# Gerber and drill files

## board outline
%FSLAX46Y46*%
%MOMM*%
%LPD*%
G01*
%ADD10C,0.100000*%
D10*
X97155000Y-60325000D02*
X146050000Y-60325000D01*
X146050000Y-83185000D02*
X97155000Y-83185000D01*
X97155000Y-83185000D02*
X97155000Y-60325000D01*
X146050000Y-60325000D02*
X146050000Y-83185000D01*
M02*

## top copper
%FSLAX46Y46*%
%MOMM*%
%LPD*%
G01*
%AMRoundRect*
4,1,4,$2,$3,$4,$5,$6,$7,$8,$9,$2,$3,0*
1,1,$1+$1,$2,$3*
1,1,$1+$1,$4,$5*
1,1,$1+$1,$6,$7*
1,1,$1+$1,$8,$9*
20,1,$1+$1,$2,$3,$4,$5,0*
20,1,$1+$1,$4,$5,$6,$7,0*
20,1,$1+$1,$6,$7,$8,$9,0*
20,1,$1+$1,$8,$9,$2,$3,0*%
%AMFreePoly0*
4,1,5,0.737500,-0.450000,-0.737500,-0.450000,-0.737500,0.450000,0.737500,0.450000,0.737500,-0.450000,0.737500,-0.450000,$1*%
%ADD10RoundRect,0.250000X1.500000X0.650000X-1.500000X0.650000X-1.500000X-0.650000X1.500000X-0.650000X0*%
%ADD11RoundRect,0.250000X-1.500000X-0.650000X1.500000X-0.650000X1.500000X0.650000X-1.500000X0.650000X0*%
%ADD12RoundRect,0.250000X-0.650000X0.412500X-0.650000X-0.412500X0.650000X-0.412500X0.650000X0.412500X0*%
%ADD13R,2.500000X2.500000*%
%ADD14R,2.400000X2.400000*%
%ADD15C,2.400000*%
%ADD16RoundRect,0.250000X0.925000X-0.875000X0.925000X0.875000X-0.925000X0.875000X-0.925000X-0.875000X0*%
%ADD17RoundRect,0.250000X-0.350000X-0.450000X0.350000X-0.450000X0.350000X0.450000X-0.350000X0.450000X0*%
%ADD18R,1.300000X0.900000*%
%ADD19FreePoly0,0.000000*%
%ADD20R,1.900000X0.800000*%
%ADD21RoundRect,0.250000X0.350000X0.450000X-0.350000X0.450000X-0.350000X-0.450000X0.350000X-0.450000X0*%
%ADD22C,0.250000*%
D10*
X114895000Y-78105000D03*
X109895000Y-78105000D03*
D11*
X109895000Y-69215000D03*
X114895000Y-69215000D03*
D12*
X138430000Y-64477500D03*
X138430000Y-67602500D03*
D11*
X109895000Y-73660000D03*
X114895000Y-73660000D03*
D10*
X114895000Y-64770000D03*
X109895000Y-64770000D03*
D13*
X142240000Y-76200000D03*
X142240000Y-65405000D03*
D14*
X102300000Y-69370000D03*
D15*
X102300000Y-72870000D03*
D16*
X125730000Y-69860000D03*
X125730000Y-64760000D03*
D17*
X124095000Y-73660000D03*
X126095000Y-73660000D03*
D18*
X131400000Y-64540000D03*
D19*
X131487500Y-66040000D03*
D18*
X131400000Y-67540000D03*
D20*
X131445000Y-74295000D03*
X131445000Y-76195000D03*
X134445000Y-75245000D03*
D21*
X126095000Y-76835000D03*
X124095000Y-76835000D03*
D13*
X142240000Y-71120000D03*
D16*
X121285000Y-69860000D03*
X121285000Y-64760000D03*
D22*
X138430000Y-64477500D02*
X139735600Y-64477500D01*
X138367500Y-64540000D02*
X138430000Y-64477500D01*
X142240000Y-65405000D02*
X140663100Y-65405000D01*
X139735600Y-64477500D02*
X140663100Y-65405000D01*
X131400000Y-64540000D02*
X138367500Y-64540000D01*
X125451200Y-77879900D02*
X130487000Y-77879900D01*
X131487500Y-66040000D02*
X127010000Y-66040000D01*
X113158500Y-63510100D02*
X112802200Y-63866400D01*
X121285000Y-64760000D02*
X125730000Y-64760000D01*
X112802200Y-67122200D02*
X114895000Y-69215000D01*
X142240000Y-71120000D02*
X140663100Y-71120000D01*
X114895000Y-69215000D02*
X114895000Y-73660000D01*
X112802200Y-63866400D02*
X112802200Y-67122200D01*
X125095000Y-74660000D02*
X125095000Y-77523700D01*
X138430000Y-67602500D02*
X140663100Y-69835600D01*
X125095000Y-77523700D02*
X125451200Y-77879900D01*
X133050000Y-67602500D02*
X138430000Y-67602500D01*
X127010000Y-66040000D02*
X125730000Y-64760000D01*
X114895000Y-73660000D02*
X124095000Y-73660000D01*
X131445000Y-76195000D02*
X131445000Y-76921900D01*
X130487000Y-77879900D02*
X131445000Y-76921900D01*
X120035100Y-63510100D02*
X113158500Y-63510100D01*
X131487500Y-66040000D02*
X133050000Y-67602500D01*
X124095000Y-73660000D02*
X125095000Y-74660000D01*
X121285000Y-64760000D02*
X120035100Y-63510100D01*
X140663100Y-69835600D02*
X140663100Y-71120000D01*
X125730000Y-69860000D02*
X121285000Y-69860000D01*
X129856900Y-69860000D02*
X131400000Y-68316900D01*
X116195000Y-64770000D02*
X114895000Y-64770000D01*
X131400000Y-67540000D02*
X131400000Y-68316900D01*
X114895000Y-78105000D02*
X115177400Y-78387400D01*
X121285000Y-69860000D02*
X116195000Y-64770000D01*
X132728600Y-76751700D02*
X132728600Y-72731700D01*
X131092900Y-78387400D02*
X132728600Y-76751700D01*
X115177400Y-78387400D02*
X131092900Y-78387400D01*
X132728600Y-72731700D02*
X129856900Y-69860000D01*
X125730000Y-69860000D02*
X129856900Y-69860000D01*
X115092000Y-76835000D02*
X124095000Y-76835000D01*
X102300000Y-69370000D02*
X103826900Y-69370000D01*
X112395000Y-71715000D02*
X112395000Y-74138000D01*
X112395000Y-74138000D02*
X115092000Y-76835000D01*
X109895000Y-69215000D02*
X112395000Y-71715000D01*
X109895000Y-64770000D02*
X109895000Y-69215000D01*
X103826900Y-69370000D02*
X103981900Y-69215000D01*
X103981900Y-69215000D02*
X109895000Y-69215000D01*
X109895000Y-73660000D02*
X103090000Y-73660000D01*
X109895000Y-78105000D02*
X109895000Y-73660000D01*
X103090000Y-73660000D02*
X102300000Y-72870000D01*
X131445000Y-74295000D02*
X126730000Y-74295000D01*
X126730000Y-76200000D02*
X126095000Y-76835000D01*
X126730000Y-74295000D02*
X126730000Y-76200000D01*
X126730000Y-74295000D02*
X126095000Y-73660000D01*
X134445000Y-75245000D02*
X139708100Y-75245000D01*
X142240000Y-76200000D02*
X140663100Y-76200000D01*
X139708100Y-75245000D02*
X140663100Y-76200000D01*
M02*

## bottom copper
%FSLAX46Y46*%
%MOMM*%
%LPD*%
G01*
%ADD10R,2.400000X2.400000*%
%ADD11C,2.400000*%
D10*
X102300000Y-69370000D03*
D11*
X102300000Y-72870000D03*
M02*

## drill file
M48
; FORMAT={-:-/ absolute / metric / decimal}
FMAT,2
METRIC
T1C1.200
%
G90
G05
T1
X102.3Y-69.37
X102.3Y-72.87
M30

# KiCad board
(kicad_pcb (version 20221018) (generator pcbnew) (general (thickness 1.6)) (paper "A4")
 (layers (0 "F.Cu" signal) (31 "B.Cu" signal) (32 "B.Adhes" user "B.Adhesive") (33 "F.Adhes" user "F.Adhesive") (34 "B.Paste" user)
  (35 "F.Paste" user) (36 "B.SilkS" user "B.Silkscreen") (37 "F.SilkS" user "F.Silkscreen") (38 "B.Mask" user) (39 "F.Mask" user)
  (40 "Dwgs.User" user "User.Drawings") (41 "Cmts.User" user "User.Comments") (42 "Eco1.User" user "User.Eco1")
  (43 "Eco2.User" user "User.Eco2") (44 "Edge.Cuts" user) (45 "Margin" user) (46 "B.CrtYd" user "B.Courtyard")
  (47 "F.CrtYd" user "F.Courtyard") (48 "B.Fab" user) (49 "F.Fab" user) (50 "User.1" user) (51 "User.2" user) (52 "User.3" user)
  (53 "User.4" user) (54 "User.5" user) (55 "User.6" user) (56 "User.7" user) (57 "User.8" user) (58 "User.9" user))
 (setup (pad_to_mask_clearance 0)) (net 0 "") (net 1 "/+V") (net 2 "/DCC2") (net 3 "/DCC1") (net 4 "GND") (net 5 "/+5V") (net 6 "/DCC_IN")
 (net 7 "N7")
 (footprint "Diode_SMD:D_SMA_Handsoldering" (layer "F.Cu") (at 112.395 78.105 180)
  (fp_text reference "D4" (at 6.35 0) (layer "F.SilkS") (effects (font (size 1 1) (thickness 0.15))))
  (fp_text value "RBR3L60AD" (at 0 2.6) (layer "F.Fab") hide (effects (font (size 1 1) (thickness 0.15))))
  (pad "1" smd roundrect (at -2.5 0 180) (size 3.5 1.8) (layers "F.Cu" "F.Paste" "F.Mask") (roundrect_rratio 0.1388888889) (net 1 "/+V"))
  (pad "2" smd roundrect (at 2.5 0 180) (size 3.5 1.8) (layers "F.Cu" "F.Paste" "F.Mask") (roundrect_rratio 0.1388888889) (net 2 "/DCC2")))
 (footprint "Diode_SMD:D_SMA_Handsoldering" (layer "F.Cu") (at 112.395 69.215)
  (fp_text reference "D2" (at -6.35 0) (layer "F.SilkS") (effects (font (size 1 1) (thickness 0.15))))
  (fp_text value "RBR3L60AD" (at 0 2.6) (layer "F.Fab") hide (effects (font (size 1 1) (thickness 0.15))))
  (pad "1" smd roundrect (at -2.5 0) (size 3.5 1.8) (layers "F.Cu" "F.Paste" "F.Mask") (roundrect_rratio 0.1388888889) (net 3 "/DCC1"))
  (pad "2" smd roundrect (at 2.5 0) (size 3.5 1.8) (layers "F.Cu" "F.Paste" "F.Mask") (roundrect_rratio 0.1388888889) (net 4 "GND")))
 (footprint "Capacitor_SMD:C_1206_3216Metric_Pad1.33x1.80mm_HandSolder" (layer "F.Cu") (at 138.43 66.04 -90)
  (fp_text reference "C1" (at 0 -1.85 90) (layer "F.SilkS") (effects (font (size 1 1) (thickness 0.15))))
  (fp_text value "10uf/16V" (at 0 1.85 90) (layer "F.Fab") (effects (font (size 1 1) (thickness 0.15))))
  (pad "1" smd roundrect (at -1.5625 0 270) (size 1.325 1.8) (layers "F.Cu" "F.Paste" "F.Mask") (roundrect_rratio 0.188679) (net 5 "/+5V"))
  (pad "2" smd roundrect (at 1.5625 0 270) (size 1.325 1.8) (layers "F.Cu" "F.Paste" "F.Mask") (roundrect_rratio 0.188679) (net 4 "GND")))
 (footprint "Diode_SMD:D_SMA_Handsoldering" (layer "F.Cu") (at 112.395 73.66)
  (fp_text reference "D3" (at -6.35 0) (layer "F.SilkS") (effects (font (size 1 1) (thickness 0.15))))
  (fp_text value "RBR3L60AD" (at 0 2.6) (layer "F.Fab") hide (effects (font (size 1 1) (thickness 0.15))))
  (pad "1" smd roundrect (at -2.5 0) (size 3.5 1.8) (layers "F.Cu" "F.Paste" "F.Mask") (roundrect_rratio 0.1388888889) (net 2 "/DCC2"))
  (pad "2" smd roundrect (at 2.5 0) (size 3.5 1.8) (layers "F.Cu" "F.Paste" "F.Mask") (roundrect_rratio 0.1388888889) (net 4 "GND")))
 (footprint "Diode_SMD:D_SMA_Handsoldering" (layer "F.Cu") (at 112.395 64.77 180)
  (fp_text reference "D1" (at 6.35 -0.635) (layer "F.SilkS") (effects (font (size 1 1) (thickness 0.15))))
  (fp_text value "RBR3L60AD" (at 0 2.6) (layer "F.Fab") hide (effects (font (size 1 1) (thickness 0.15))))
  (pad "1" smd roundrect (at -2.5 0 180) (size 3.5 1.8) (layers "F.Cu" "F.Paste" "F.Mask") (roundrect_rratio 0.1388888889) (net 1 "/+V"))
  (pad "2" smd roundrect (at 2.5 0 180) (size 3.5 1.8) (layers "F.Cu" "F.Paste" "F.Mask") (roundrect_rratio 0.1388888889) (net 3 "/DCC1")))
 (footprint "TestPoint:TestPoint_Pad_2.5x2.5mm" (layer "F.Cu") (at 142.24 76.2)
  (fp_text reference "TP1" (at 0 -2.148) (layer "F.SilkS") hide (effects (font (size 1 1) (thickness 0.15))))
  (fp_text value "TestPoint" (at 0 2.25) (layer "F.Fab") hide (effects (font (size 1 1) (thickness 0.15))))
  (pad "1" smd rect (at 0 0) (size 2.5 2.5) (layers "F.Cu" "F.Mask") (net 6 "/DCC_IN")))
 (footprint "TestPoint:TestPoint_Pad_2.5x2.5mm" (layer "F.Cu") (at 142.24 65.405)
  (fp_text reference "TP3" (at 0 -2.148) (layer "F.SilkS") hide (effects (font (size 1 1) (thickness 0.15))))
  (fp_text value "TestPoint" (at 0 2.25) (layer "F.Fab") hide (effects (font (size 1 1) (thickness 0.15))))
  (pad "1" smd rect (at 0 0) (size 2.5 2.5) (layers "F.Cu" "F.Mask") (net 5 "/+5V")))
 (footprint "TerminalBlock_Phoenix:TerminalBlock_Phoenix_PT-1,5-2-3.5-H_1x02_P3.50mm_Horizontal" (layer "F.Cu") (at 102.3 69.37 -90)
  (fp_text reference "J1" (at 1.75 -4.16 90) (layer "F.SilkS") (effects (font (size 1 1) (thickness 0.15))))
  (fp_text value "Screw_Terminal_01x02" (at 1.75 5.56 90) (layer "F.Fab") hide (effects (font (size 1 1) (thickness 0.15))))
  (pad "1" thru_hole rect (at 0 0 270) (size 2.4 2.4) (drill 1.2) (layers "*.Cu" "*.Mask") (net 3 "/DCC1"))
  (pad "2" thru_hole circle (at 3.5 0 270) (size 2.4 2.4) (drill 1.2) (layers "*.Cu" "*.Mask") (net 2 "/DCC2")))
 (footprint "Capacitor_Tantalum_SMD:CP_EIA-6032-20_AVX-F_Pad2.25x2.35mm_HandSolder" (layer "F.Cu") (at 125.73 67.31 90)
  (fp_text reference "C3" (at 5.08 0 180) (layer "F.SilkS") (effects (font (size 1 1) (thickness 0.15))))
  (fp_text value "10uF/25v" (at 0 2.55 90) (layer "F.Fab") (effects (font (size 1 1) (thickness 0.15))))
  (pad "1" smd roundrect (at -2.55 0 90) (size 2.25 2.35) (layers "F.Cu" "F.Paste" "F.Mask") (roundrect_rratio 0.111111) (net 1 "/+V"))
  (pad "2" smd roundrect (at 2.55 0 90) (size 2.25 2.35) (layers "F.Cu" "F.Paste" "F.Mask") (roundrect_rratio 0.111111) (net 4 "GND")))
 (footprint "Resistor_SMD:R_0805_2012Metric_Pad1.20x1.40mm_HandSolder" (layer "F.Cu") (at 125.095 73.66)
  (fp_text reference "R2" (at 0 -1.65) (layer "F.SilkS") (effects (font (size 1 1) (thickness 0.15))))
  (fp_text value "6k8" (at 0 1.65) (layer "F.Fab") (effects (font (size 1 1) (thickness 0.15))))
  (pad "1" smd roundrect (at -1 0) (size 1.2 1.4) (layers "F.Cu" "F.Paste" "F.Mask") (roundrect_rratio 0.208333) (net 4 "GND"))
  (pad "2" smd roundrect (at 1 0) (size 1.2 1.4) (layers "F.Cu" "F.Paste" "F.Mask") (roundrect_rratio 0.208333) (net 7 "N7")))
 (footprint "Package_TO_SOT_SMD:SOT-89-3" (layer "F.Cu") (at 133.35 66.04)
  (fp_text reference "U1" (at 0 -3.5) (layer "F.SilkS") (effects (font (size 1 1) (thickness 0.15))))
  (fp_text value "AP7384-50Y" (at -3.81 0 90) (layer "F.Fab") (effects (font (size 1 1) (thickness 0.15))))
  (pad "1" smd rect (at -1.95 -1.5) (size 1.3 0.9) (layers "F.Cu" "F.Paste" "F.Mask") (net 5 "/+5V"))
  (pad "2" smd custom (at -1.8625 0) (size 1.475 0.9) (layers "F.Cu" "F.Paste" "F.Mask") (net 4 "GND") (zone_connect 2)
   (thermal_bridge_angle 45) (options (clearance outline) (anchor rect)) (primitives))
  (pad "3" smd rect (at -1.95 1.5) (size 1.3 0.9) (layers "F.Cu" "F.Paste" "F.Mask") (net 1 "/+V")))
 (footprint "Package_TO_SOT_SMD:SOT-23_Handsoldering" (layer "F.Cu") (at 132.945 75.245)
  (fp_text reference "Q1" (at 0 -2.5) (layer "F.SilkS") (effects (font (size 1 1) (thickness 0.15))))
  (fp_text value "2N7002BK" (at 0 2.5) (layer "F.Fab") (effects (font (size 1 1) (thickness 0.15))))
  (pad "1" smd rect (at -1.5 -0.95) (size 1.9 0.8) (layers "F.Cu" "F.Paste" "F.Mask") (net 7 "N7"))
  (pad "2" smd rect (at -1.5 0.95) (size 1.9 0.8) (layers "F.Cu" "F.Paste" "F.Mask") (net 4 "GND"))
  (pad "3" smd rect (at 1.5 0) (size 1.9 0.8) (layers "F.Cu" "F.Paste" "F.Mask") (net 6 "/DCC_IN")))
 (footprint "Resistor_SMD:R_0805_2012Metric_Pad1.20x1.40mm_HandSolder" (layer "F.Cu") (at 125.095 76.835 180)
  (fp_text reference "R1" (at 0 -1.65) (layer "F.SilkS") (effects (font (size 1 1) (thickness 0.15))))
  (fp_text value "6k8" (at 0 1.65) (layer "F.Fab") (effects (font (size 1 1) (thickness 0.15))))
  (pad "1" smd roundrect (at -1 0 180) (size 1.2 1.4) (layers "F.Cu" "F.Paste" "F.Mask") (roundrect_rratio 0.208333) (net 7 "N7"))
  (pad "2" smd roundrect (at 1 0 180) (size 1.2 1.4) (layers "F.Cu" "F.Paste" "F.Mask") (roundrect_rratio 0.208333) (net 3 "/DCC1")))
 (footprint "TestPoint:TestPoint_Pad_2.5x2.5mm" (layer "F.Cu") (at 142.24 71.12)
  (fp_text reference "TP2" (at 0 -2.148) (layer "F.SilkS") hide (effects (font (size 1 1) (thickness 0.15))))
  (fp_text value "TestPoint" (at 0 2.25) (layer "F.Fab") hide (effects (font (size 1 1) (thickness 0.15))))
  (pad "1" smd rect (at 0 0) (size 2.5 2.5) (layers "F.Cu" "F.Mask") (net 4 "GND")))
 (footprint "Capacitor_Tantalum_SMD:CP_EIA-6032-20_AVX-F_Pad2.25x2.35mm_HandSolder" (layer "F.Cu") (at 121.285 67.31 90)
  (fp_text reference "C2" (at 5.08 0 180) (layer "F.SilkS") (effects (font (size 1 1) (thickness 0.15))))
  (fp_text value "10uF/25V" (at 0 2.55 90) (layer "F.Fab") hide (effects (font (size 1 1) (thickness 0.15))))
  (pad "1" smd roundrect (at -2.55 0 90) (size 2.25 2.35) (layers "F.Cu" "F.Paste" "F.Mask") (roundrect_rratio 0.111111) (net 1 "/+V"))
  (pad "2" smd roundrect (at 2.55 0 90) (size 2.25 2.35) (layers "F.Cu" "F.Paste" "F.Mask") (roundrect_rratio 0.111111) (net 4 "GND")))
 (gr_line (start 97.155 60.325) (end 146.05 60.325) (stroke (width 0.1) (type default)) (layer "Edge.Cuts"))
 (gr_line (start 146.05 83.185) (end 97.155 83.185) (stroke (width 0.1) (type default)) (layer "Edge.Cuts"))
 (gr_line (start 97.155 83.185) (end 97.155 60.325) (stroke (width 0.1) (type default)) (layer "Edge.Cuts"))
 (gr_line (start 146.05 60.325) (end 146.05 83.185) (stroke (width 0.1) (type default)) (layer "Edge.Cuts"))
 (segment (start 138.43 64.4775) (end 139.7356 64.4775) (width 0.25) (layer "F.Cu") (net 5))
 (segment (start 138.3675 64.54) (end 138.43 64.4775) (width 0.25) (layer "F.Cu") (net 5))
 (segment (start 142.24 65.405) (end 140.6631 65.405) (width 0.25) (layer "F.Cu") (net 5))
 (segment (start 139.7356 64.4775) (end 140.6631 65.405) (width 0.25) (layer "F.Cu") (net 5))
 (segment (start 131.4 64.54) (end 138.3675 64.54) (width 0.25) (layer "F.Cu") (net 5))
 (segment (start 125.4512 77.8799) (end 130.487 77.8799) (width 0.25) (layer "F.Cu") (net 4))
 (segment (start 131.4875 66.04) (end 127.01 66.04) (width 0.25) (layer "F.Cu") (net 4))
 (segment (start 113.1585 63.5101) (end 112.8022 63.8664) (width 0.25) (layer "F.Cu") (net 4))
 (segment (start 121.285 64.76) (end 125.73 64.76) (width 0.25) (layer "F.Cu") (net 4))
 (segment (start 112.8022 67.1222) (end 114.895 69.215) (width 0.25) (layer "F.Cu") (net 4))
 (segment (start 142.24 71.12) (end 140.6631 71.12) (width 0.25) (layer "F.Cu") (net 4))
 (segment (start 114.895 69.215) (end 114.895 73.66) (width 0.25) (layer "F.Cu") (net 4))
 (segment (start 112.8022 63.8664) (end 112.8022 67.1222) (width 0.25) (layer "F.Cu") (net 4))
 (segment (start 125.095 74.66) (end 125.095 77.5237) (width 0.25) (layer "F.Cu") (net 4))
 (segment (start 138.43 67.6025) (end 140.6631 69.8356) (width 0.25) (layer "F.Cu") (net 4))
 (segment (start 125.095 77.5237) (end 125.4512 77.8799) (width 0.25) (layer "F.Cu") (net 4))
 (segment (start 133.05 67.6025) (end 138.43 67.6025) (width 0.25) (layer "F.Cu") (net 4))
 (segment (start 127.01 66.04) (end 125.73 64.76) (width 0.25) (layer "F.Cu") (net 4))
 (segment (start 114.895 73.66) (end 124.095 73.66) (width 0.25) (layer "F.Cu") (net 4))
 (segment (start 131.445 76.195) (end 131.445 76.9219) (width 0.25) (layer "F.Cu") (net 4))
 (segment (start 130.487 77.8799) (end 131.445 76.9219) (width 0.25) (layer "F.Cu") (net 4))
 (segment (start 120.0351 63.5101) (end 113.1585 63.5101) (width 0.25) (layer "F.Cu") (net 4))
 (segment (start 131.4875 66.04) (end 133.05 67.6025) (width 0.25) (layer "F.Cu") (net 4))
 (segment (start 124.095 73.66) (end 125.095 74.66) (width 0.25) (layer "F.Cu") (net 4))
 (segment (start 121.285 64.76) (end 120.0351 63.5101) (width 0.25) (layer "F.Cu") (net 4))
 (segment (start 140.6631 69.8356) (end 140.6631 71.12) (width 0.25) (layer "F.Cu") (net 4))
 (segment (start 125.73 69.86) (end 121.285 69.86) (width 0.25) (layer "F.Cu") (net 1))
 (segment (start 129.8569 69.86) (end 131.4 68.3169) (width 0.25) (layer "F.Cu") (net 1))
 (segment (start 116.195 64.77) (end 114.895 64.77) (width 0.25) (layer "F.Cu") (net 1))
 (segment (start 131.4 67.54) (end 131.4 68.3169) (width 0.25) (layer "F.Cu") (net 1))
 (segment (start 114.895 78.105) (end 115.1774 78.3874) (width 0.25) (layer "F.Cu") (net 1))
 (segment (start 121.285 69.86) (end 116.195 64.77) (width 0.25) (layer "F.Cu") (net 1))
 (segment (start 132.7286 76.7517) (end 132.7286 72.7317) (width 0.25) (layer "F.Cu") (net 1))
 (segment (start 131.0929 78.3874) (end 132.7286 76.7517) (width 0.25) (layer "F.Cu") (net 1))
 (segment (start 115.1774 78.3874) (end 131.0929 78.3874) (width 0.25) (layer "F.Cu") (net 1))
 (segment (start 132.7286 72.7317) (end 129.8569 69.86) (width 0.25) (layer "F.Cu") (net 1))
 (segment (start 125.73 69.86) (end 129.8569 69.86) (width 0.25) (layer "F.Cu") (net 1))
 (segment (start 115.092 76.835) (end 124.095 76.835) (width 0.25) (layer "F.Cu") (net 3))
 (segment (start 102.3 69.37) (end 103.8269 69.37) (width 0.25) (layer "F.Cu") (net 3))
 (segment (start 112.395 71.715) (end 112.395 74.138) (width 0.25) (layer "F.Cu") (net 3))
 (segment (start 112.395 74.138) (end 115.092 76.835) (width 0.25) (layer "F.Cu") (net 3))
 (segment (start 109.895 69.215) (end 112.395 71.715) (width 0.25) (layer "F.Cu") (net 3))
 (segment (start 109.895 64.77) (end 109.895 69.215) (width 0.25) (layer "F.Cu") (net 3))
 (segment (start 103.8269 69.37) (end 103.9819 69.215) (width 0.25) (layer "F.Cu") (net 3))
 (segment (start 103.9819 69.215) (end 109.895 69.215) (width 0.25) (layer "F.Cu") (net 3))
 (segment (start 109.895 73.66) (end 103.09 73.66) (width 0.25) (layer "F.Cu") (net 2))
 (segment (start 109.895 78.105) (end 109.895 73.66) (width 0.25) (layer "F.Cu") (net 2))
 (segment (start 103.09 73.66) (end 102.3 72.87) (width 0.25) (layer "F.Cu") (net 2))
 (segment (start 131.445 74.295) (end 126.73 74.295) (width 0.25) (layer "F.Cu") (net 7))
 (segment (start 126.73 76.2) (end 126.095 76.835) (width 0.25) (layer "F.Cu") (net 7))
 (segment (start 126.73 74.295) (end 126.73 76.2) (width 0.25) (layer "F.Cu") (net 7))
 (segment (start 126.73 74.295) (end 126.095 73.66) (width 0.25) (layer "F.Cu") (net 7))
 (segment (start 134.445 75.245) (end 139.7081 75.245) (width 0.25) (layer "F.Cu") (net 6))
 (segment (start 142.24 76.2) (end 140.6631 76.2) (width 0.25) (layer "F.Cu") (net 6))
 (segment (start 139.7081 75.245) (end 140.6631 76.2) (width 0.25) (layer "F.Cu") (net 6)))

